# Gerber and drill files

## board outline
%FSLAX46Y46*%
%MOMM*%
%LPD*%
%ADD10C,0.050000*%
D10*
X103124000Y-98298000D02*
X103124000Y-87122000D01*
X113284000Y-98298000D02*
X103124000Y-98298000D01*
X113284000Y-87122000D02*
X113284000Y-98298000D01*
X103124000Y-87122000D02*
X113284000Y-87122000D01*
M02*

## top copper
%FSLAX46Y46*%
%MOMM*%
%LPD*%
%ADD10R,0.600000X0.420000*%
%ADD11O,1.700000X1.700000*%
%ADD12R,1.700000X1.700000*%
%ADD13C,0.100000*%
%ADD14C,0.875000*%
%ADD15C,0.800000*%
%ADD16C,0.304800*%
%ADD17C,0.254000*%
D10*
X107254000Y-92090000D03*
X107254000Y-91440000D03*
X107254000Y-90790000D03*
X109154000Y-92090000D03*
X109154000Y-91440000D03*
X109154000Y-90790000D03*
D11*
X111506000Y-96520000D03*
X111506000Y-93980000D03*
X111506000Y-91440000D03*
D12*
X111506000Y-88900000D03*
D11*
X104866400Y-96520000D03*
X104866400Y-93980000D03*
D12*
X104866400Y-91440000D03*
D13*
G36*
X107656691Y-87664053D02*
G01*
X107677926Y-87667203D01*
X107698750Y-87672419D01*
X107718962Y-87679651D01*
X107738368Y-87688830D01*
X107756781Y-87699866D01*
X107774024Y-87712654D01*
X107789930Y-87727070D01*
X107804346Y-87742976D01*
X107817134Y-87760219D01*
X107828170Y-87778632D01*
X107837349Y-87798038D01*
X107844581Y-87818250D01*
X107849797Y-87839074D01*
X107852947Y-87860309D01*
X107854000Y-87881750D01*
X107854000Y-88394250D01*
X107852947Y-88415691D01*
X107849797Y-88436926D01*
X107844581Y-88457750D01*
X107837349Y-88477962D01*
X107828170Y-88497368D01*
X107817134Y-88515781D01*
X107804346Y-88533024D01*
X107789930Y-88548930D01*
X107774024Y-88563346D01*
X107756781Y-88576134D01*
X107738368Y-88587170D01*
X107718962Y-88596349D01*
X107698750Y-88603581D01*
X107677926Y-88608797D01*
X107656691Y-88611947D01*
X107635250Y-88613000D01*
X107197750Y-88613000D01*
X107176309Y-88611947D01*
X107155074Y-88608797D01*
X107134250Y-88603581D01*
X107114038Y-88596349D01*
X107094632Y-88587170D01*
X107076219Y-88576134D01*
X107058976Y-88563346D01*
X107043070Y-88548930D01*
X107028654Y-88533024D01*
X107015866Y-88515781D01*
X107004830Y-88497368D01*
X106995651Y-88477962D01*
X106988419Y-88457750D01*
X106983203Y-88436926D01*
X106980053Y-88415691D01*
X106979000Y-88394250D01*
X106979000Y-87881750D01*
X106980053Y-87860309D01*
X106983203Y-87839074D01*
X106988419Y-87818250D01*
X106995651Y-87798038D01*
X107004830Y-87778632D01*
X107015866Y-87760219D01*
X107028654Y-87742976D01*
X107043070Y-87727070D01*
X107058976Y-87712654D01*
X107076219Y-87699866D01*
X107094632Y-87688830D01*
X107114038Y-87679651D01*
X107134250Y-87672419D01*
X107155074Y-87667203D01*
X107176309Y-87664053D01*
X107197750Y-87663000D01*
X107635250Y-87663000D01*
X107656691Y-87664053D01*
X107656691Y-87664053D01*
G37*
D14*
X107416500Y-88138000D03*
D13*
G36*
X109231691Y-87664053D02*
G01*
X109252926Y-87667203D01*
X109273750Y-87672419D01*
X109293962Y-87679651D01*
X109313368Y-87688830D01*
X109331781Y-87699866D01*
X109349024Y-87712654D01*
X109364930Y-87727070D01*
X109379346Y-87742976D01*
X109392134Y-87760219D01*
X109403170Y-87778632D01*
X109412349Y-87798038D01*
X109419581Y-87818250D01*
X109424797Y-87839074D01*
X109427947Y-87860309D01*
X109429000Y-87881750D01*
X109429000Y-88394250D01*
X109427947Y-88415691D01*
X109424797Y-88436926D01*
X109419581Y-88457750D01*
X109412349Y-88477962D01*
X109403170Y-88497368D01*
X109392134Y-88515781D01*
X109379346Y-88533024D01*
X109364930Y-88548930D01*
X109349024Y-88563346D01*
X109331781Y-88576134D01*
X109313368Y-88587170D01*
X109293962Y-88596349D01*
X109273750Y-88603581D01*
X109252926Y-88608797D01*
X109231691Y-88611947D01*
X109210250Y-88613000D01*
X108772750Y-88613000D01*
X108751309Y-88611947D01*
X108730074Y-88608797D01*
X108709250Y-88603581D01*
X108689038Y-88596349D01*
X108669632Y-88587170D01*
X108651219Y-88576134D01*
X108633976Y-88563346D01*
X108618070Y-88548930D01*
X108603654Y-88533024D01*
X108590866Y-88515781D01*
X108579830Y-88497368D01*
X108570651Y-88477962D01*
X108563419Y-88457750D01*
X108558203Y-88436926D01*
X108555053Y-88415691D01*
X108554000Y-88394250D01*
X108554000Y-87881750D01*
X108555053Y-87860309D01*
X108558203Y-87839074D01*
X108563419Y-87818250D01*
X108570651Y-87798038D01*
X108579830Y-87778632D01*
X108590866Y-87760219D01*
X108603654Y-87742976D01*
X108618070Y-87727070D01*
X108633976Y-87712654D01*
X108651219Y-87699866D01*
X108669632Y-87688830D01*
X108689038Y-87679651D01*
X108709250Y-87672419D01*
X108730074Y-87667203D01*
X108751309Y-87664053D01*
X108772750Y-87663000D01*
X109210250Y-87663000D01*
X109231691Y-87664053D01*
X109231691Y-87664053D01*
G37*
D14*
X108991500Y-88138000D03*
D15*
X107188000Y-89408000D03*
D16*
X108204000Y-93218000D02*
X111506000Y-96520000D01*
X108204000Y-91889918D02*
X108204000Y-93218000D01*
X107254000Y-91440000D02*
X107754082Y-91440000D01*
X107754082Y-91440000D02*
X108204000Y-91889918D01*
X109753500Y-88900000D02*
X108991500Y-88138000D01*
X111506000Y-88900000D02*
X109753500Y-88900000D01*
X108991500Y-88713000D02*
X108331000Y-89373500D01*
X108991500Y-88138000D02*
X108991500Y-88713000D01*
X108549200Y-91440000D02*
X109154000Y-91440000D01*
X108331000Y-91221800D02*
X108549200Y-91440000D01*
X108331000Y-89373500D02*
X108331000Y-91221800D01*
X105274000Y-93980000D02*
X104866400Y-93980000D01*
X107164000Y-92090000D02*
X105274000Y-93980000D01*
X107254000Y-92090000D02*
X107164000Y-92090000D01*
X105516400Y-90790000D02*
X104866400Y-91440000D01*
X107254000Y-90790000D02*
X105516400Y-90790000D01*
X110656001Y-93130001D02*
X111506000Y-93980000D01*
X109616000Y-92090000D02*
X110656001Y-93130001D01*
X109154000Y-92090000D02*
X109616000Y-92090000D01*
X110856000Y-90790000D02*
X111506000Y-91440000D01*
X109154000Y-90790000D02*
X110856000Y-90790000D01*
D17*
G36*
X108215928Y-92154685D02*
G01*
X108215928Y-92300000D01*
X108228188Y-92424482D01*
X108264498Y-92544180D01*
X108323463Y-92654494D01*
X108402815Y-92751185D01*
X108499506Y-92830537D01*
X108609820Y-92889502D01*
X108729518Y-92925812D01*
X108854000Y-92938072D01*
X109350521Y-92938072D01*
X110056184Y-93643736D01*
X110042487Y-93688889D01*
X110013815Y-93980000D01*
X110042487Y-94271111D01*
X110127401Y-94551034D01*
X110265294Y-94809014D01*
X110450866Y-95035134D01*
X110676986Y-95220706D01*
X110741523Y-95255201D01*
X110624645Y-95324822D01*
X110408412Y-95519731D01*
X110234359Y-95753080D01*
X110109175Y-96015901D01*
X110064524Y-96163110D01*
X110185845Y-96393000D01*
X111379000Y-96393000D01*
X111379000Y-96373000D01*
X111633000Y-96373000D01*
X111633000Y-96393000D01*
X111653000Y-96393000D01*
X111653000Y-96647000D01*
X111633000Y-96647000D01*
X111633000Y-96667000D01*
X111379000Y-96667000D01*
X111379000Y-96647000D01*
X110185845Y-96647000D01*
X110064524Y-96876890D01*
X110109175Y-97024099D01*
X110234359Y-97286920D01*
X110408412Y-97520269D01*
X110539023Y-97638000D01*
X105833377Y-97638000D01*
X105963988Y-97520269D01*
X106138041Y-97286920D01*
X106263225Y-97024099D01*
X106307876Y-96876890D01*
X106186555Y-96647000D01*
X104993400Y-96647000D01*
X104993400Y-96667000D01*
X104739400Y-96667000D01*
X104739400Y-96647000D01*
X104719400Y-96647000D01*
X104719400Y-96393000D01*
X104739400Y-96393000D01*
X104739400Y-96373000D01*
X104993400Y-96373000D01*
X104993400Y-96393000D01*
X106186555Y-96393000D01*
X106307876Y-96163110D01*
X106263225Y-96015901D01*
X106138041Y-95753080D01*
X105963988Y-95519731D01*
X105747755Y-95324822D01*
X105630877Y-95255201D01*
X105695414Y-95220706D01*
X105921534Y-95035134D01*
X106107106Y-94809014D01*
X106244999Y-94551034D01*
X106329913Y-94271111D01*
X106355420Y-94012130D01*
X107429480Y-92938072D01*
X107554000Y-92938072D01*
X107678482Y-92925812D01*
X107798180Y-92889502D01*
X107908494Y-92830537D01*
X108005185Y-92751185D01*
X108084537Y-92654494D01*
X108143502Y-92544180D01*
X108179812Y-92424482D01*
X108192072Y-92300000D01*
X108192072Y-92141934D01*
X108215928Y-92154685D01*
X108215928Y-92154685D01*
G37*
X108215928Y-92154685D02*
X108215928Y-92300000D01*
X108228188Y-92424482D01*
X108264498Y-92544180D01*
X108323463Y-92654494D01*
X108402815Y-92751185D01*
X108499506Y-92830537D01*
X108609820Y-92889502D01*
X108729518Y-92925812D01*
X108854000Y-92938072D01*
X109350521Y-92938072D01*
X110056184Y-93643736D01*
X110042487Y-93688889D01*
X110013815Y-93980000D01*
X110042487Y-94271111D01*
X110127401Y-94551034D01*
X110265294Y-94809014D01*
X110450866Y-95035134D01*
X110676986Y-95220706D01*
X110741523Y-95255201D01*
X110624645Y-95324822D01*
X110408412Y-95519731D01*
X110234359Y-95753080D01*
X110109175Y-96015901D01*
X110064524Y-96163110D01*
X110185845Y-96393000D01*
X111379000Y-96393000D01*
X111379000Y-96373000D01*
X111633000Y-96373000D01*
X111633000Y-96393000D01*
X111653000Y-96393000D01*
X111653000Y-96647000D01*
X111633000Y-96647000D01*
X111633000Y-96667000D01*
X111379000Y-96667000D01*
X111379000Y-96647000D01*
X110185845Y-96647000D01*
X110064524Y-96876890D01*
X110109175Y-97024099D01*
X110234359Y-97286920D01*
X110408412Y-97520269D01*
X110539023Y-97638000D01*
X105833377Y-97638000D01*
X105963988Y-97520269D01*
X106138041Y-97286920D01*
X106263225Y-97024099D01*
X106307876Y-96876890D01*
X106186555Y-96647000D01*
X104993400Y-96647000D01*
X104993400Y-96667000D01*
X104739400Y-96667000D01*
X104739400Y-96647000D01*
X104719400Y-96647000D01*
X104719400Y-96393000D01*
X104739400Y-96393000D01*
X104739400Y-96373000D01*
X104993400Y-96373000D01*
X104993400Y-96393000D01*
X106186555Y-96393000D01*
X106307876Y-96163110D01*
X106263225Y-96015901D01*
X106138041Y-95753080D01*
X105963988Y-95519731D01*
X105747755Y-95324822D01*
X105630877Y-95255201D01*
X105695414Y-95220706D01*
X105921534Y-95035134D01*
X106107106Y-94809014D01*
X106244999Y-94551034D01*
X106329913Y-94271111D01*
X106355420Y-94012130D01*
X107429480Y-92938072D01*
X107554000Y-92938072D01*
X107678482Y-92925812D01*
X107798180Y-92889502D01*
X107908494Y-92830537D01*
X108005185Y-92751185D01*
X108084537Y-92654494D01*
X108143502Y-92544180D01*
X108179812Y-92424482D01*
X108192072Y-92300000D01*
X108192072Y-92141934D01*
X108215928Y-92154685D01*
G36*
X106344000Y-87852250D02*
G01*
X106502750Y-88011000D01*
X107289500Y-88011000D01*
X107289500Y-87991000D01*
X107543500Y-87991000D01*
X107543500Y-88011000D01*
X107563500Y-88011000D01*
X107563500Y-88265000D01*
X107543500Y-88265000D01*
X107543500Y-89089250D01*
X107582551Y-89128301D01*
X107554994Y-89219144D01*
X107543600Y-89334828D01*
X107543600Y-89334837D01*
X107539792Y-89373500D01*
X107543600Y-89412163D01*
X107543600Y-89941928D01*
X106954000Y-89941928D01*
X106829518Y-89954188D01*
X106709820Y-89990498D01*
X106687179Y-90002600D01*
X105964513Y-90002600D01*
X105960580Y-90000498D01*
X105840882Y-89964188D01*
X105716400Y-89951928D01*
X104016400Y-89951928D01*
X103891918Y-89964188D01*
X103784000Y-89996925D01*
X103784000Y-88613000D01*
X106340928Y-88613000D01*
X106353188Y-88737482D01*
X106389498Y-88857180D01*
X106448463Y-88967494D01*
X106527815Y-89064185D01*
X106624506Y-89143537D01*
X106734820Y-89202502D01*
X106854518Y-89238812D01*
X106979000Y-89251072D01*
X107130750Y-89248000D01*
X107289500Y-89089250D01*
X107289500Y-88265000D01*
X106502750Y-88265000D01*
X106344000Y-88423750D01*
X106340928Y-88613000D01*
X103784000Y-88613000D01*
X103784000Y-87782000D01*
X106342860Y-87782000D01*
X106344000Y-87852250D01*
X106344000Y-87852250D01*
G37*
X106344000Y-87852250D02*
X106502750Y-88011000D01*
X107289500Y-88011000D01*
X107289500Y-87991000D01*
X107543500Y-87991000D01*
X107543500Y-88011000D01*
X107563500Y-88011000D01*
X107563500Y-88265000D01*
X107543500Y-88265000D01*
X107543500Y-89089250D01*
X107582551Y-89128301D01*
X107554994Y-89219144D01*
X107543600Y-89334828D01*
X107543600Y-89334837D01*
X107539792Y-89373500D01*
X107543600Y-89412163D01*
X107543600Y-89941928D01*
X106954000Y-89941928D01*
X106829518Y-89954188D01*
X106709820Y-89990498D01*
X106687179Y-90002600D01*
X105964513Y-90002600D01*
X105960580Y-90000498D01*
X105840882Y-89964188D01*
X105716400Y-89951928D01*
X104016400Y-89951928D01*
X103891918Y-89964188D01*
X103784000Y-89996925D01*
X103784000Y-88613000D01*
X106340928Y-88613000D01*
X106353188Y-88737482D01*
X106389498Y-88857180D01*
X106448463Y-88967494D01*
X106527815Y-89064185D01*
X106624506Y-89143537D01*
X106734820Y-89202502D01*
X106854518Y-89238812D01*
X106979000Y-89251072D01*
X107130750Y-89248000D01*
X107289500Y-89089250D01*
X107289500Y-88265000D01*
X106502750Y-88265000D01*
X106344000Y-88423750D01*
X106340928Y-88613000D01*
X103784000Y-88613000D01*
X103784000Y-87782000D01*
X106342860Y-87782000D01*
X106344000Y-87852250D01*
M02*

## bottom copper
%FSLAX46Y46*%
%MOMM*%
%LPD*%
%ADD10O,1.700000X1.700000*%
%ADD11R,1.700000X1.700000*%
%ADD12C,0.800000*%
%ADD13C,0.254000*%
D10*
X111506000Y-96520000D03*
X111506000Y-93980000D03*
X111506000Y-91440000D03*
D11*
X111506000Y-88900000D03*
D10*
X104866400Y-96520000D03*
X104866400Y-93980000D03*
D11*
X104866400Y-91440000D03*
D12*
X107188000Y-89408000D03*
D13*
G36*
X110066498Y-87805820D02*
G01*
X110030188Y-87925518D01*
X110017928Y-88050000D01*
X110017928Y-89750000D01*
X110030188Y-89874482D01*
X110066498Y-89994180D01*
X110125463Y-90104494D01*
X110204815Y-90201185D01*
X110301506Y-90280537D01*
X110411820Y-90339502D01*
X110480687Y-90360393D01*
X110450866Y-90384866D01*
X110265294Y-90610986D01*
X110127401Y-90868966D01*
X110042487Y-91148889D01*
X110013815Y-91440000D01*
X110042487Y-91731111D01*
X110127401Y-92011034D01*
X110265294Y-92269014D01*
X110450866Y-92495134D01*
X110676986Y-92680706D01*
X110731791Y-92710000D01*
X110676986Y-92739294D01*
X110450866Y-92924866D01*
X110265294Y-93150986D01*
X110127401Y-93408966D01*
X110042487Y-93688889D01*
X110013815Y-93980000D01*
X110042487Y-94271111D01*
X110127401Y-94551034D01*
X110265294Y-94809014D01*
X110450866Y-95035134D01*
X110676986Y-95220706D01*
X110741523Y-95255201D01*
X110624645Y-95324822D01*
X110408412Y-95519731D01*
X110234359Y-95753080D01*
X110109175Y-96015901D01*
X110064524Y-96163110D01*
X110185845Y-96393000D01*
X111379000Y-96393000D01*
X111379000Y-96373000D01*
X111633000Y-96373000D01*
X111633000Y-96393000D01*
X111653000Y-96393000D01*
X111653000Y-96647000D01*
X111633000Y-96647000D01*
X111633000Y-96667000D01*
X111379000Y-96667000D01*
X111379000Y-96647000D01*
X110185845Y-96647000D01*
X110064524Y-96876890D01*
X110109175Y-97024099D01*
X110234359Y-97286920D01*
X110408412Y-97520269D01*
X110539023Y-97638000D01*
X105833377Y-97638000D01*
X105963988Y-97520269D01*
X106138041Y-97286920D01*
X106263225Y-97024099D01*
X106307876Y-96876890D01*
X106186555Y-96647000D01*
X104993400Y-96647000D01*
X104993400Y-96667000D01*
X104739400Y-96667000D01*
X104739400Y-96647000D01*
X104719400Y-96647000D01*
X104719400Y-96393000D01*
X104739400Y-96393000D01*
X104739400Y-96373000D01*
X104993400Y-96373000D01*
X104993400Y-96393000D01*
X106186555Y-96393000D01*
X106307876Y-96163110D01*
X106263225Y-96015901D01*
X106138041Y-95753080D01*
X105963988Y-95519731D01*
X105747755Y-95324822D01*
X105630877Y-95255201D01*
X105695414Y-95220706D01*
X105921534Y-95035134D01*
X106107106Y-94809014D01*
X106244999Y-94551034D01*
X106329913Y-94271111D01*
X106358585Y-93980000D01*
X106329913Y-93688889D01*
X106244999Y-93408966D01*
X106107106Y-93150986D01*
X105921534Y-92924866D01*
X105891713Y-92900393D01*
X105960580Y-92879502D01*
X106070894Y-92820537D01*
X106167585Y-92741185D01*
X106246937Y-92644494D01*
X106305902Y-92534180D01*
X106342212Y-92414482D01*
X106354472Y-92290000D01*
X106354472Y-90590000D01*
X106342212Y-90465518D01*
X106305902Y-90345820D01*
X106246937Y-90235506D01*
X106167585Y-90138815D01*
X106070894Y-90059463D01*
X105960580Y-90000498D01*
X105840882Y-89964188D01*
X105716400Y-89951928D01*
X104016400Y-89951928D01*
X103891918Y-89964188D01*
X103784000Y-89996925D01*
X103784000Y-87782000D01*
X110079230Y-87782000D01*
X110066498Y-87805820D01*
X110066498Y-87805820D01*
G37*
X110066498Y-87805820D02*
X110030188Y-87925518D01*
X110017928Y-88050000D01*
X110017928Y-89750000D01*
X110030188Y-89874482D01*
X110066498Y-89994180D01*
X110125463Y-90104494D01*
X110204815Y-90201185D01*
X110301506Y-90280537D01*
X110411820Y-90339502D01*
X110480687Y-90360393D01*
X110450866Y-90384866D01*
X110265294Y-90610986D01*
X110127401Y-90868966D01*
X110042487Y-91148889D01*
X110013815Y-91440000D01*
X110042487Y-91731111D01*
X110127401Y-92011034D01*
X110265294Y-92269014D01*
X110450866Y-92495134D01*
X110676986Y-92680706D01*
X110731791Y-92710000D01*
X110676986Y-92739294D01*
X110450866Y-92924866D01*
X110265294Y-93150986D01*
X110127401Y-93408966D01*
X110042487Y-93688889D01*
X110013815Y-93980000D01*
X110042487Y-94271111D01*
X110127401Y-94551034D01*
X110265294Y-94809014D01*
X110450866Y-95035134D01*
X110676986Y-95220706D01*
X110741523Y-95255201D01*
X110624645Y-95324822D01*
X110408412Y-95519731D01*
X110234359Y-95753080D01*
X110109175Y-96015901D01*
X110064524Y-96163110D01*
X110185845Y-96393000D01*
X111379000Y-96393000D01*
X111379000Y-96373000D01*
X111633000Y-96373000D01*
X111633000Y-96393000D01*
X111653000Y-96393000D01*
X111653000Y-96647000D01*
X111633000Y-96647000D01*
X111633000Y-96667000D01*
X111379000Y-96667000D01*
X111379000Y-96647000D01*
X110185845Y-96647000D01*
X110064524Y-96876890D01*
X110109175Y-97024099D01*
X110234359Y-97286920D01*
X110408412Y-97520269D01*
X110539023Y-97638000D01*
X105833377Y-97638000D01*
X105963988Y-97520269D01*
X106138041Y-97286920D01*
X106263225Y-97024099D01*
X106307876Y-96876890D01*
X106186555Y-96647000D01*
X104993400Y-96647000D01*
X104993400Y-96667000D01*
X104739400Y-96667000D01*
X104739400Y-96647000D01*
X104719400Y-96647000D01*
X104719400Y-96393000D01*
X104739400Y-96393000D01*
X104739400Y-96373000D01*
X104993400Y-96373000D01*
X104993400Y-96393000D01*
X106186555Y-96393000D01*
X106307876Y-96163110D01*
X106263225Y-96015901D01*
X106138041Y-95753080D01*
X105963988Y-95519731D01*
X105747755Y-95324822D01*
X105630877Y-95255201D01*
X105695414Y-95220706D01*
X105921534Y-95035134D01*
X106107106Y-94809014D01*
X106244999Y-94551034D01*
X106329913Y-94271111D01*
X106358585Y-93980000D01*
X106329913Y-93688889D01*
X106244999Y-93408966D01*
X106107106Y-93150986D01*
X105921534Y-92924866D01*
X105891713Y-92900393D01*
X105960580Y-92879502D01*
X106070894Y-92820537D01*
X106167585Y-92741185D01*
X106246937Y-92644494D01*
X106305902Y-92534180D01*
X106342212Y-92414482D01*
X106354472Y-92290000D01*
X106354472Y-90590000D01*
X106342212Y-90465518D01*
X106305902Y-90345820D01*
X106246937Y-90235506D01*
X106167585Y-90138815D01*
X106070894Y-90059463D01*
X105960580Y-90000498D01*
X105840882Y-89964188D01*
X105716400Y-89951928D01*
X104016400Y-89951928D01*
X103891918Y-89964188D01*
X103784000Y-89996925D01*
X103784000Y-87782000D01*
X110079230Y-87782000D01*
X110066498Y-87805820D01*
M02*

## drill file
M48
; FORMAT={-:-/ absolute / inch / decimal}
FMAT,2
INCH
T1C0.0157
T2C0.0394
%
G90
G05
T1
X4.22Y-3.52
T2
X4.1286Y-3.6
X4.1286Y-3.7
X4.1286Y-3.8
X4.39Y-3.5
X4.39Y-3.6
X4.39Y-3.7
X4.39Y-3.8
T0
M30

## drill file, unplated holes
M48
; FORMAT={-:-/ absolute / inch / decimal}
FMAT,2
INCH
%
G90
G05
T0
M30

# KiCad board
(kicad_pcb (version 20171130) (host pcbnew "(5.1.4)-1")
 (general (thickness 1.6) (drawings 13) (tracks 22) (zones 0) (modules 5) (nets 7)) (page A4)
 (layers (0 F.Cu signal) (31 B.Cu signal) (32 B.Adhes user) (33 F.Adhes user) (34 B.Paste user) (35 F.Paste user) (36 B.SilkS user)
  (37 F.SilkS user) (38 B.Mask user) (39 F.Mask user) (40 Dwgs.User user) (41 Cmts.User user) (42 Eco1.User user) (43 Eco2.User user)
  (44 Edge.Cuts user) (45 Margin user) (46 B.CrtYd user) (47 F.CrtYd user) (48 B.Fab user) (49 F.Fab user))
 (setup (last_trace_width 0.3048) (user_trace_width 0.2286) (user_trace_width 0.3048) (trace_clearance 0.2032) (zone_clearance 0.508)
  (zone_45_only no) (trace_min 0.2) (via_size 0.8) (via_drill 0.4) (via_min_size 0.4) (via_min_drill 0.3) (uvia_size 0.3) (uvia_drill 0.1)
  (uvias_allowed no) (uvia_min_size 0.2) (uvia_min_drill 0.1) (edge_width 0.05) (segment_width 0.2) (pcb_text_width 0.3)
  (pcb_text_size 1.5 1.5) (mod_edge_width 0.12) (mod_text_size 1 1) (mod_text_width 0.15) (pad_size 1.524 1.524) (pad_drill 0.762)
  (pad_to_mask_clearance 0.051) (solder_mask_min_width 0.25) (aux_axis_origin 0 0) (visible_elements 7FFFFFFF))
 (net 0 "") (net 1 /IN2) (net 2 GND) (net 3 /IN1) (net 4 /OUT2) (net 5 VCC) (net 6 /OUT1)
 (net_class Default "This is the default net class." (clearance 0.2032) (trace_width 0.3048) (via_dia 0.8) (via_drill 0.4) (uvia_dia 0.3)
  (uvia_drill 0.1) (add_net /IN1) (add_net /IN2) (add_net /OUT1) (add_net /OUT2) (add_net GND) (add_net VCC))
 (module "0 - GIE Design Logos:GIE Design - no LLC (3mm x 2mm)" (layer F.Cu) (at 104.902 88.392)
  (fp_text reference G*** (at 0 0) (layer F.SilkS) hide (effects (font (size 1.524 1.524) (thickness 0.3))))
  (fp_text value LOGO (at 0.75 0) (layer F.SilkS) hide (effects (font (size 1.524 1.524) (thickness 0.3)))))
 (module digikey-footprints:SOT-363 (layer F.Cu) (at 108.204 91.44 270)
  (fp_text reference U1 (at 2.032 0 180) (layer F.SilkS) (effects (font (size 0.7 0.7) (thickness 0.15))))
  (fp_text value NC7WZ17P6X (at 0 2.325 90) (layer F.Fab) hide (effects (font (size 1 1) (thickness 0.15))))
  (pad 3 smd rect (at 0.65 0.95 270) (size 0.42 0.6) (layers F.Cu F.Paste F.Mask) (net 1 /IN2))
  (pad 2 smd rect (at 0 0.95 270) (size 0.42 0.6) (layers F.Cu F.Paste F.Mask) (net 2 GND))
  (pad 1 smd rect (at -0.65 0.95 270) (size 0.42 0.6) (layers F.Cu F.Paste F.Mask) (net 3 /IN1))
  (pad 4 smd rect (at 0.65 -0.95 270) (size 0.42 0.6) (layers F.Cu F.Paste F.Mask) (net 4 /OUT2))
  (pad 5 smd rect (at 0 -0.95 270) (size 0.42 0.6) (layers F.Cu F.Paste F.Mask) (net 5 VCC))
  (pad 6 smd rect (at -0.65 -0.95 270) (size 0.42 0.6) (layers F.Cu F.Paste F.Mask) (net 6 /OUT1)))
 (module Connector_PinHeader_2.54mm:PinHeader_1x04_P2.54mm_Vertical (layer F.Cu) (at 111.506 88.9)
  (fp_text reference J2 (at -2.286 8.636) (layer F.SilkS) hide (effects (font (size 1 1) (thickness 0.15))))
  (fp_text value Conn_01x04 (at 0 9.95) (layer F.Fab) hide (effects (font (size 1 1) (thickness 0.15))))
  (pad 4 thru_hole oval (at 0 7.62) (size 1.7 1.7) (drill 1) (layers *.Cu *.Mask) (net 2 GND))
  (pad 3 thru_hole oval (at 0 5.08) (size 1.7 1.7) (drill 1) (layers *.Cu *.Mask) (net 4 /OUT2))
  (pad 2 thru_hole oval (at 0 2.54) (size 1.7 1.7) (drill 1) (layers *.Cu *.Mask) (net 6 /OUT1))
  (pad 1 thru_hole rect (at 0 0) (size 1.7 1.7) (drill 1) (layers *.Cu *.Mask) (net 5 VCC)))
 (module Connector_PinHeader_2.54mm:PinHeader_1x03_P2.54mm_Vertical (layer F.Cu) (at 104.8664 91.44)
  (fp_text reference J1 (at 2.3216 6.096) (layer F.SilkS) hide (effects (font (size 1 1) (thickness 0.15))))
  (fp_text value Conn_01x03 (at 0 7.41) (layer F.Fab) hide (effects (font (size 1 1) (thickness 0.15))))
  (pad 3 thru_hole oval (at 0 5.08) (size 1.7 1.7) (drill 1) (layers *.Cu *.Mask) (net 2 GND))
  (pad 2 thru_hole oval (at 0 2.54) (size 1.7 1.7) (drill 1) (layers *.Cu *.Mask) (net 1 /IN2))
  (pad 1 thru_hole rect (at 0 0) (size 1.7 1.7) (drill 1) (layers *.Cu *.Mask) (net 3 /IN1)))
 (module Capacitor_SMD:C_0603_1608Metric (layer F.Cu) (at 108.204 88.138 180)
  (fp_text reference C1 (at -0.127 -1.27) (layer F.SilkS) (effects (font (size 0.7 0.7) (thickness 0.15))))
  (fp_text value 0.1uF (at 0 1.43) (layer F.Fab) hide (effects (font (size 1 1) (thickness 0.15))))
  (pad 2 smd roundrect (at 0.7875 0 180) (size 0.875 0.95) (layers F.Cu F.Paste F.Mask) (roundrect_rratio 0.25) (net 2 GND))
  (pad 1 smd roundrect (at -0.7875 0 180) (size 0.875 0.95) (layers F.Cu F.Paste F.Mask) (roundrect_rratio 0.25) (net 5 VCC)))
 (gr_line (start 103.124 98.298) (end 103.124 87.122) (layer Edge.Cuts) (width 0.05))
 (gr_line (start 113.284 98.298) (end 103.124 98.298) (layer Edge.Cuts) (width 0.05))
 (gr_line (start 113.284 87.122) (end 113.284 98.298) (layer Edge.Cuts) (width 0.05))
 (gr_line (start 103.124 87.122) (end 113.284 87.122) (layer Edge.Cuts) (width 0.05))
 (segment (start 108.204 93.218) (end 111.506 96.52) (width 0.3048) (layer F.Cu) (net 2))
 (segment (start 108.204 91.889918) (end 108.204 93.218) (width 0.3048) (layer F.Cu) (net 2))
 (segment (start 107.254 91.44) (end 107.754082 91.44) (width 0.3048) (layer F.Cu) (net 2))
 (segment (start 107.754082 91.44) (end 108.204 91.889918) (width 0.3048) (layer F.Cu) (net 2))
 (via (at 107.188 89.408) (size 0.8) (drill 0.4) (layers F.Cu B.Cu) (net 2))
 (segment (start 109.7535 88.9) (end 108.9915 88.138) (width 0.3048) (layer F.Cu) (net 5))
 (segment (start 111.506 88.9) (end 109.7535 88.9) (width 0.3048) (layer F.Cu) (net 5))
 (segment (start 108.9915 88.713) (end 108.331 89.3735) (width 0.3048) (layer F.Cu) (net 5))
 (segment (start 108.9915 88.138) (end 108.9915 88.713) (width 0.3048) (layer F.Cu) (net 5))
 (segment (start 108.5492 91.44) (end 109.154 91.44) (width 0.3048) (layer F.Cu) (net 5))
 (segment (start 108.331 91.2218) (end 108.5492 91.44) (width 0.3048) (layer F.Cu) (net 5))
 (segment (start 108.331 89.3735) (end 108.331 91.2218) (width 0.3048) (layer F.Cu) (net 5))
 (segment (start 105.274 93.98) (end 104.8664 93.98) (width 0.3048) (layer F.Cu) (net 1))
 (segment (start 107.164 92.09) (end 105.274 93.98) (width 0.3048) (layer F.Cu) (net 1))
 (segment (start 107.254 92.09) (end 107.164 92.09) (width 0.3048) (layer F.Cu) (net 1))
 (segment (start 105.5164 90.79) (end 104.8664 91.44) (width 0.3048) (layer F.Cu) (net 3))
 (segment (start 107.254 90.79) (end 105.5164 90.79) (width 0.3048) (layer F.Cu) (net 3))
 (segment (start 110.656001 93.130001) (end 111.506 93.98) (width 0.3048) (layer F.Cu) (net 4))
 (segment (start 109.616 92.09) (end 110.656001 93.130001) (width 0.3048) (layer F.Cu) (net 4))
 (segment (start 109.154 92.09) (end 109.616 92.09) (width 0.3048) (layer F.Cu) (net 4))
 (segment (start 110.856 90.79) (end 111.506 91.44) (width 0.3048) (layer F.Cu) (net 6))
 (segment (start 109.154 90.79) (end 110.856 90.79) (width 0.3048) (layer F.Cu) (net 6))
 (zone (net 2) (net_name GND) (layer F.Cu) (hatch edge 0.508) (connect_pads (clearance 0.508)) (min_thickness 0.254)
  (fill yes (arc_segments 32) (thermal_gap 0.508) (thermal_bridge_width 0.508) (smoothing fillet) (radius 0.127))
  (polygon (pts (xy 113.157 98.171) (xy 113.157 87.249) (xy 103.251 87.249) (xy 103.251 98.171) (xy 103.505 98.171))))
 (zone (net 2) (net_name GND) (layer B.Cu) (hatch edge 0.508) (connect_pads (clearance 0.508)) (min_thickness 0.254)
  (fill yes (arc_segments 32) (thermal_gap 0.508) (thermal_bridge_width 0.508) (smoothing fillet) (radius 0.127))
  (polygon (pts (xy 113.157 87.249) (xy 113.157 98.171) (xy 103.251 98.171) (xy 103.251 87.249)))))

